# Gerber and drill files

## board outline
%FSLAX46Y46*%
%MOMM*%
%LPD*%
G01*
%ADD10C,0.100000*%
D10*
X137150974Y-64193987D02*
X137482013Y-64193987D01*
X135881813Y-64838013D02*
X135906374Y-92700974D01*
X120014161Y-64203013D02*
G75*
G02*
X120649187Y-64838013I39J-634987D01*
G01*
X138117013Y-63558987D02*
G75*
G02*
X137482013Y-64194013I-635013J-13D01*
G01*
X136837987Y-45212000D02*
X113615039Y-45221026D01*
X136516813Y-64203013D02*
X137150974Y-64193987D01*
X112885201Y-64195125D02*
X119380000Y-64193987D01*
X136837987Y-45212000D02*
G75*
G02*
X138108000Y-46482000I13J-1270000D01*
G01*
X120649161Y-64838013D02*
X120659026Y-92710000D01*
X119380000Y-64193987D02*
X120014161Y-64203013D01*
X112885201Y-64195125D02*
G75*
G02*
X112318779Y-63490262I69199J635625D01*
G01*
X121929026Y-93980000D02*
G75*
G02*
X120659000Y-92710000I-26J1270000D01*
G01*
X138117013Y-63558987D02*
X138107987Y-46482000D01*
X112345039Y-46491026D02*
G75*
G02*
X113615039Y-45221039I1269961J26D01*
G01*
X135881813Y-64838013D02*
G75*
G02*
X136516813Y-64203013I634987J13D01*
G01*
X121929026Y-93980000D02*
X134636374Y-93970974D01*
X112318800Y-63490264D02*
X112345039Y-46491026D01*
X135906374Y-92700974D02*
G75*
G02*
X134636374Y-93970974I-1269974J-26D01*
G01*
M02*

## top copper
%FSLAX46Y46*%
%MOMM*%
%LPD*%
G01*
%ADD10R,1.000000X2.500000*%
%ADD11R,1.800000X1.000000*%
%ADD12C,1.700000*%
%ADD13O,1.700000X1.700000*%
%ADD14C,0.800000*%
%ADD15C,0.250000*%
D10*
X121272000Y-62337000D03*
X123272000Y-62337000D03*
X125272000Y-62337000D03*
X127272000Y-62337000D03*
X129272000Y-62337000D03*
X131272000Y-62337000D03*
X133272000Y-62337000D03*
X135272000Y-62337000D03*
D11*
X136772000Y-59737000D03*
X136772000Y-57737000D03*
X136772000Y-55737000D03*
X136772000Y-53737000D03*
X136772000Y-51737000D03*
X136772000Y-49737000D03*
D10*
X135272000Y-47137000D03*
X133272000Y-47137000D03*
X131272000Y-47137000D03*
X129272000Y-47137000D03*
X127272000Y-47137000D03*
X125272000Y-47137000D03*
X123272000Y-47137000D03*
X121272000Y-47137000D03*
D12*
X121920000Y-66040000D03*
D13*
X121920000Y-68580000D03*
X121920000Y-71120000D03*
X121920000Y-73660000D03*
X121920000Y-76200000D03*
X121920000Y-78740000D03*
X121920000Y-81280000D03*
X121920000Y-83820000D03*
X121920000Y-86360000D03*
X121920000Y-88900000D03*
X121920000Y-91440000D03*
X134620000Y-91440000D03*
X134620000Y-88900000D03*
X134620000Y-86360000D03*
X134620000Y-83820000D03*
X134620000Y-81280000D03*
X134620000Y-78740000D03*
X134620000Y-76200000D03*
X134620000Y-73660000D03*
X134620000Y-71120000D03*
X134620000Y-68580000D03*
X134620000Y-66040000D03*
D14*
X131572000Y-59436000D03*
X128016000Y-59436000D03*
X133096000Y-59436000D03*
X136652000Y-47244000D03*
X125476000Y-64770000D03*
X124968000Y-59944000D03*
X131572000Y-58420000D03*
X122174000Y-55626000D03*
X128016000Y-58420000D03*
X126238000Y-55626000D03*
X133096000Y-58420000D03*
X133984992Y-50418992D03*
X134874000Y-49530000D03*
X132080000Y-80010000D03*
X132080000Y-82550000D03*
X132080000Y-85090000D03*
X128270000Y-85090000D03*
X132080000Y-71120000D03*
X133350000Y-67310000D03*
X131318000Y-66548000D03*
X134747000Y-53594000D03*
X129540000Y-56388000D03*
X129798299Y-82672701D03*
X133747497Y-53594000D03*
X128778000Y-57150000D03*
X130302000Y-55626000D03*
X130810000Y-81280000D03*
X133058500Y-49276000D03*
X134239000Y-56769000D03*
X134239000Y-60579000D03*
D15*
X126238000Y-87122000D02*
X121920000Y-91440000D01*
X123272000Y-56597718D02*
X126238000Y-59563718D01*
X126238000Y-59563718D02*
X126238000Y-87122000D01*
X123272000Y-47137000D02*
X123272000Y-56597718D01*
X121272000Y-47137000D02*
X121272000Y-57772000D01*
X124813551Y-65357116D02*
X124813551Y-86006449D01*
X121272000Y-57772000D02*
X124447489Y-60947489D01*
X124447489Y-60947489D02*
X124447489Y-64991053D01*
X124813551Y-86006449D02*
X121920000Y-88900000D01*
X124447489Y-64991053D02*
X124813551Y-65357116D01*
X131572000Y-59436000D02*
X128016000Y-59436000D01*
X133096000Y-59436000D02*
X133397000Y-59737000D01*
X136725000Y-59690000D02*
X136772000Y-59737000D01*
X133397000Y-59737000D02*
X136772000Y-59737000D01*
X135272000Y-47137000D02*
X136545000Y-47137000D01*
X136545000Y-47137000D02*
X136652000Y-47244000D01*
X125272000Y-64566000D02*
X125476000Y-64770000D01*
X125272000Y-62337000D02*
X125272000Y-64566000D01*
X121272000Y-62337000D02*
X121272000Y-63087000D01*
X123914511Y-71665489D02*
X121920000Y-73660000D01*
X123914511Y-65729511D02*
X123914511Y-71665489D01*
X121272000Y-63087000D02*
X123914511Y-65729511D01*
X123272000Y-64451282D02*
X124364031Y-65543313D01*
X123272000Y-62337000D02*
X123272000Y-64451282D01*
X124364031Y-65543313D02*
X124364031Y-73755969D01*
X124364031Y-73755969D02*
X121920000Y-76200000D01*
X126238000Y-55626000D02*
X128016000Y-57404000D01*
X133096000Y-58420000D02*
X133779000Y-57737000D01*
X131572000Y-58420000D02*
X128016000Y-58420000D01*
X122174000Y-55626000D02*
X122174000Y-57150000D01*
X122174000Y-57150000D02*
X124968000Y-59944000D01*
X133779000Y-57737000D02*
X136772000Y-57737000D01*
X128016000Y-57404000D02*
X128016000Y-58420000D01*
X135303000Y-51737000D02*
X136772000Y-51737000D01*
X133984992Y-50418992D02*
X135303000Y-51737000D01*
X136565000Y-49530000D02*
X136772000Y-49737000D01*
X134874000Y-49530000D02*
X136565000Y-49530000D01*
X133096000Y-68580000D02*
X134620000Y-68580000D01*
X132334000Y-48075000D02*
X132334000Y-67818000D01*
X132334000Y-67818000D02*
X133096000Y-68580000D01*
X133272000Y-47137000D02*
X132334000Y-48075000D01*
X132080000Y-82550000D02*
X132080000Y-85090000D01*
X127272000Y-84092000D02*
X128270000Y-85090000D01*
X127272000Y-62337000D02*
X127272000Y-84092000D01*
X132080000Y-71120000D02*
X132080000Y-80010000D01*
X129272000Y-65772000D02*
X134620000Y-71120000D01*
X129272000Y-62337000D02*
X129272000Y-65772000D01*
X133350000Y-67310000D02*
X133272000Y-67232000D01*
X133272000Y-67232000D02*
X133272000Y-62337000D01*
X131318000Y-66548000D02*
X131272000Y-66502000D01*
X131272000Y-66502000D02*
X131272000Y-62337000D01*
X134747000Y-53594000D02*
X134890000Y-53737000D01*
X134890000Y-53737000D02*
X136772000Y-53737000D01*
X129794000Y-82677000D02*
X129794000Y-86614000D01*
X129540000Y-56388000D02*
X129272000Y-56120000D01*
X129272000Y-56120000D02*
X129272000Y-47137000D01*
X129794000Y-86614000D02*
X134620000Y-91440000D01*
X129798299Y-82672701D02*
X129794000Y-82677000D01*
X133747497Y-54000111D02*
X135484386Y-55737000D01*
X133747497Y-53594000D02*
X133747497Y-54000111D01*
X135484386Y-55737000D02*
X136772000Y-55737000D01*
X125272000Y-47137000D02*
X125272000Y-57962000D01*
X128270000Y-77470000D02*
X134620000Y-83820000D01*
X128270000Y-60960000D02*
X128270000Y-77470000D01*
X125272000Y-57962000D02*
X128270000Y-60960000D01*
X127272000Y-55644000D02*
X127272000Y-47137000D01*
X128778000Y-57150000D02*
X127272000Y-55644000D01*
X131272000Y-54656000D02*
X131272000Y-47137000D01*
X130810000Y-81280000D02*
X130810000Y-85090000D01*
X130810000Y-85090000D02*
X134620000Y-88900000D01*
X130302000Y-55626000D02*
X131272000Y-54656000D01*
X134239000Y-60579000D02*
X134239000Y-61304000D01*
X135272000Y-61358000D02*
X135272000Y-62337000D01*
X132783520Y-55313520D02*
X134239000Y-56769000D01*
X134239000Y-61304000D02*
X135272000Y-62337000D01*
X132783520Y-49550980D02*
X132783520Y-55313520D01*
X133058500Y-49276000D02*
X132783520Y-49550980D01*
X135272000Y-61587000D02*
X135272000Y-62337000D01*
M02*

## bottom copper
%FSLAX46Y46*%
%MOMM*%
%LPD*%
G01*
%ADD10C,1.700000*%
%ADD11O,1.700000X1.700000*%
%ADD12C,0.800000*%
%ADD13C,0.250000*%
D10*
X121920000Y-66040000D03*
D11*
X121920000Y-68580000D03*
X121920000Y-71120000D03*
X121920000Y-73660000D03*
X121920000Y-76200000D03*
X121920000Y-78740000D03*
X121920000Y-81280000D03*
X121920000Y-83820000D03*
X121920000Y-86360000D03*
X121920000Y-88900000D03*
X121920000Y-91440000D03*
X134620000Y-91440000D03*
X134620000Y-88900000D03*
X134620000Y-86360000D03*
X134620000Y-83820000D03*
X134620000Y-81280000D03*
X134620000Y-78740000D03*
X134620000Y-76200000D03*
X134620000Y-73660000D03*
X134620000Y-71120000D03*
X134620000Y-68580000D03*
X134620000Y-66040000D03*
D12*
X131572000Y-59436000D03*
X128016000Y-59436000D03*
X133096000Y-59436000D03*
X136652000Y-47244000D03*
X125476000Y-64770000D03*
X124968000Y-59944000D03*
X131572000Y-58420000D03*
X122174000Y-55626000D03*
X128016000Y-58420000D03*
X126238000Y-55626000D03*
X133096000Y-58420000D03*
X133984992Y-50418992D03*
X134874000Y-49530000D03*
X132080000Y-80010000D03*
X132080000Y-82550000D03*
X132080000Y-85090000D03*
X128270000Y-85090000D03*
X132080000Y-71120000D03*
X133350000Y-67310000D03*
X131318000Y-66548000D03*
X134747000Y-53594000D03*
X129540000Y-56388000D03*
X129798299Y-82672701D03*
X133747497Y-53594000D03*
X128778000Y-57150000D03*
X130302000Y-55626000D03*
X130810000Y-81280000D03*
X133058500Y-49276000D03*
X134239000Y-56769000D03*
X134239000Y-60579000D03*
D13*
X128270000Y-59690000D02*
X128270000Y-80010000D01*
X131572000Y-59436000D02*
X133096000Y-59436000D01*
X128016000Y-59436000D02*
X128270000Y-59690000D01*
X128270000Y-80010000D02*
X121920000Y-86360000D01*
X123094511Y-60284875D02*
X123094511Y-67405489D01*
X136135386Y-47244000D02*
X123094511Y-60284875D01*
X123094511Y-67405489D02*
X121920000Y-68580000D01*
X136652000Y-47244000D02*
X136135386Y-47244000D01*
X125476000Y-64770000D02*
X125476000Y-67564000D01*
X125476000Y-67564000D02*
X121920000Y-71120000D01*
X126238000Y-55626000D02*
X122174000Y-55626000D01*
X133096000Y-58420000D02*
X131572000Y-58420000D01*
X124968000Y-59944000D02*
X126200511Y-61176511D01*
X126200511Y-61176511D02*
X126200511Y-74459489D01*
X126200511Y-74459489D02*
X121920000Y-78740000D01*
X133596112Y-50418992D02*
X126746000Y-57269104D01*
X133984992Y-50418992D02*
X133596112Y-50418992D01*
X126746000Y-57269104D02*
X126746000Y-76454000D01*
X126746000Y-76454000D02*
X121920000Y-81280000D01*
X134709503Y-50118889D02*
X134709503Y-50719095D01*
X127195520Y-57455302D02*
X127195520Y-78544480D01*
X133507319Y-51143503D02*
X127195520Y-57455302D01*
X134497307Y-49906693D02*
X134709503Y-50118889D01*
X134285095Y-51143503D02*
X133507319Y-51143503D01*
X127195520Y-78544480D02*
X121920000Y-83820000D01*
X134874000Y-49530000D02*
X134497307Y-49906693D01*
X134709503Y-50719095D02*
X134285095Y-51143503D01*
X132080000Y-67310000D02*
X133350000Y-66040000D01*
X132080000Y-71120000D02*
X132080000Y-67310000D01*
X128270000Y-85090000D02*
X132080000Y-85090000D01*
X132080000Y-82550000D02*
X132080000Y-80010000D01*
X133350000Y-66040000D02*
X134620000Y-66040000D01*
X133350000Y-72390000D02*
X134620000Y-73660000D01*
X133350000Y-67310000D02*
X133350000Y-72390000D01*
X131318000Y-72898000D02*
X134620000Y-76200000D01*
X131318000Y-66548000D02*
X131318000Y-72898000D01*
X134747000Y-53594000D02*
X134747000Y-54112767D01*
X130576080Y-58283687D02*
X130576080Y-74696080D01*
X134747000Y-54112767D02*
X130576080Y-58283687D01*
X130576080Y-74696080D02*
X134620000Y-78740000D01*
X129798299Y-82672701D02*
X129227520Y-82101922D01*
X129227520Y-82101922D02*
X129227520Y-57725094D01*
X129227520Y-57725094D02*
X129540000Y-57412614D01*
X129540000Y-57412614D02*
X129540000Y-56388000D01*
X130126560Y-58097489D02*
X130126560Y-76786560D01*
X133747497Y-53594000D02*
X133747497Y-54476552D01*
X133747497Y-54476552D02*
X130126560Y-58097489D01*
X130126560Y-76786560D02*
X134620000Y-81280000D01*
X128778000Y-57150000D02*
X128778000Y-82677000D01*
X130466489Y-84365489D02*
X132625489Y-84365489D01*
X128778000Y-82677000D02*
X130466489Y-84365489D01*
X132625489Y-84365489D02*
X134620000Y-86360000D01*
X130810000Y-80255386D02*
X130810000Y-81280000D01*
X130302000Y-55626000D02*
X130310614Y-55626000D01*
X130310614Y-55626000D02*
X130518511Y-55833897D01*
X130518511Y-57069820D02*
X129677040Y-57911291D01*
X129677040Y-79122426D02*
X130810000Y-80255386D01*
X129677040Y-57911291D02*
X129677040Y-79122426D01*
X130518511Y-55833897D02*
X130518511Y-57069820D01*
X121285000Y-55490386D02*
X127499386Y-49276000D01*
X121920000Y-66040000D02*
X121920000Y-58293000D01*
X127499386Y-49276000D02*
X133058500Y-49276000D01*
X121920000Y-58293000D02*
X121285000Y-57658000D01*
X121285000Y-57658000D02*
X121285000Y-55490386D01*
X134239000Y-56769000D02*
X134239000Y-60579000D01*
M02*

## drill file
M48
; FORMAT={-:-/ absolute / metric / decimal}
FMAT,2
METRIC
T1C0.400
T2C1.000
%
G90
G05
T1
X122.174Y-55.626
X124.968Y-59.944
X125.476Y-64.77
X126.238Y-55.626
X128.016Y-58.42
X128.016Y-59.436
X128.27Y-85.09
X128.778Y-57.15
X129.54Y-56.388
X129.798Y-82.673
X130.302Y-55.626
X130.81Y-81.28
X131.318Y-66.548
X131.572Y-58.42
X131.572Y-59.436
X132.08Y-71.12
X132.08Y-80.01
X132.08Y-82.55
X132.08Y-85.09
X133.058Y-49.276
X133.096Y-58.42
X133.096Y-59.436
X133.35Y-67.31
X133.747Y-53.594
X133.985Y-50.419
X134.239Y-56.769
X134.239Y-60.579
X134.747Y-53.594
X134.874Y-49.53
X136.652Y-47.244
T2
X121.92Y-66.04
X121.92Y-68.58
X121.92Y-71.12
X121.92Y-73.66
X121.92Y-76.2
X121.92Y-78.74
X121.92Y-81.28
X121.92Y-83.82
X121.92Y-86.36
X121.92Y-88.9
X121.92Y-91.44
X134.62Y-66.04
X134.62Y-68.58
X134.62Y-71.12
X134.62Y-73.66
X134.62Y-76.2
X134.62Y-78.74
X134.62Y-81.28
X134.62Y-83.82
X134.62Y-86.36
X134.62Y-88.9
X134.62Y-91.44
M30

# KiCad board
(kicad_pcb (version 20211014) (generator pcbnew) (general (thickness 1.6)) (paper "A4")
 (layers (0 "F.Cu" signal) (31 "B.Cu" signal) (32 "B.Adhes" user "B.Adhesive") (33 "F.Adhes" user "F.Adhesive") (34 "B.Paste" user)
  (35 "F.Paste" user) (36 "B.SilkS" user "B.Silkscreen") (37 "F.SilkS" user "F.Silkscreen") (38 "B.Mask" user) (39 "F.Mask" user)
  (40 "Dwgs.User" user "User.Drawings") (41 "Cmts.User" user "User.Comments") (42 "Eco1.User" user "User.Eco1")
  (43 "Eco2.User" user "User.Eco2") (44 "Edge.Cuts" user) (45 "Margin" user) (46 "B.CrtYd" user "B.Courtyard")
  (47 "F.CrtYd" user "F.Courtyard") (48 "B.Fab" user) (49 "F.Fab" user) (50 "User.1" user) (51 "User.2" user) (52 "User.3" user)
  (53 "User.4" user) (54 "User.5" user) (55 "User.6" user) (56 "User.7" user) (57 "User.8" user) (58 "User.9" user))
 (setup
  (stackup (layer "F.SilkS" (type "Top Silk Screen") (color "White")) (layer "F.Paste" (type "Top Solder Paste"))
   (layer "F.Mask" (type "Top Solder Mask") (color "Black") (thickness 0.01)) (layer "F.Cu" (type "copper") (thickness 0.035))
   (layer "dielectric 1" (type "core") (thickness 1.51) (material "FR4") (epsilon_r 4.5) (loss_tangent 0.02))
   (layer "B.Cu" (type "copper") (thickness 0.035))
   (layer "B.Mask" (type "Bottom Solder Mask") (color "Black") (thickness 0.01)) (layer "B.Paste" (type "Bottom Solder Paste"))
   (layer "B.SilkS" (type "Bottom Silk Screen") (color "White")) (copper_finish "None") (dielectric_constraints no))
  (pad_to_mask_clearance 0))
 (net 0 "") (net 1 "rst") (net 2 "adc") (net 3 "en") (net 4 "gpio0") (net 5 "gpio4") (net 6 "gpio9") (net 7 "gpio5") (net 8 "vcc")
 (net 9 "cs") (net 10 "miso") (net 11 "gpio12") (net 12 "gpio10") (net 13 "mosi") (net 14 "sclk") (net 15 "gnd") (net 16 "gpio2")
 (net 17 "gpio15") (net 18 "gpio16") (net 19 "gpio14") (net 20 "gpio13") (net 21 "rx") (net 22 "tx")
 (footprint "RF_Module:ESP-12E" (layer "F.Cu") (at 124.772 54.737 90)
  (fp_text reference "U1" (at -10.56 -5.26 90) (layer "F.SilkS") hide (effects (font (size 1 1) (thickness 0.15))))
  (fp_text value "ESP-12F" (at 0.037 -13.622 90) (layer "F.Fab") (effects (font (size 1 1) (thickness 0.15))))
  (pad "1" smd rect (at -7.6 -3.5 90) (size 2.5 1) (layers "F.Cu" "F.Paste" "F.Mask") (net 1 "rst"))
  (pad "2" smd rect (at -7.6 -1.5 90) (size 2.5 1) (layers "F.Cu" "F.Paste" "F.Mask") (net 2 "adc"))
  (pad "3" smd rect (at -7.6 0.5 90) (size 2.5 1) (layers "F.Cu" "F.Paste" "F.Mask") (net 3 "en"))
  (pad "4" smd rect (at -7.6 2.5 90) (size 2.5 1) (layers "F.Cu" "F.Paste" "F.Mask") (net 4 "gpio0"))
  (pad "5" smd rect (at -7.6 4.5 90) (size 2.5 1) (layers "F.Cu" "F.Paste" "F.Mask") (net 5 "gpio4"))
  (pad "6" smd rect (at -7.6 6.5 90) (size 2.5 1) (layers "F.Cu" "F.Paste" "F.Mask") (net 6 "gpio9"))
  (pad "7" smd rect (at -7.6 8.5 90) (size 2.5 1) (layers "F.Cu" "F.Paste" "F.Mask") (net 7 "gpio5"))
  (pad "8" smd rect (at -7.6 10.5 90) (size 2.5 1) (layers "F.Cu" "F.Paste" "F.Mask") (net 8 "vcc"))
  (pad "9" smd rect (at -5 12 90) (size 1 1.8) (layers "F.Cu" "F.Paste" "F.Mask") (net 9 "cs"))
  (pad "10" smd rect (at -3 12 90) (size 1 1.8) (layers "F.Cu" "F.Paste" "F.Mask") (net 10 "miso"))
  (pad "11" smd rect (at -1 12 90) (size 1 1.8) (layers "F.Cu" "F.Paste" "F.Mask") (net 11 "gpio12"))
  (pad "12" smd rect (at 1 12 90) (size 1 1.8) (layers "F.Cu" "F.Paste" "F.Mask") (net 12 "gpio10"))
  (pad "13" smd rect (at 3 12 90) (size 1 1.8) (layers "F.Cu" "F.Paste" "F.Mask") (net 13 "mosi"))
  (pad "14" smd rect (at 5 12 90) (size 1 1.8) (layers "F.Cu" "F.Paste" "F.Mask") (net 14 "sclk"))
  (pad "15" smd rect (at 7.6 10.5 90) (size 2.5 1) (layers "F.Cu" "F.Paste" "F.Mask") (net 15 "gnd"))
  (pad "16" smd rect (at 7.6 8.5 90) (size 2.5 1) (layers "F.Cu" "F.Paste" "F.Mask") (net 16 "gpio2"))
  (pad "17" smd rect (at 7.6 6.5 90) (size 2.5 1) (layers "F.Cu" "F.Paste" "F.Mask") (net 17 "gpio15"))
  (pad "18" smd rect (at 7.6 4.5 90) (size 2.5 1) (layers "F.Cu" "F.Paste" "F.Mask") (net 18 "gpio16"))
  (pad "19" smd rect (at 7.6 2.5 90) (size 2.5 1) (layers "F.Cu" "F.Paste" "F.Mask") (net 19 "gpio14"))
  (pad "20" smd rect (at 7.6 0.5 90) (size 2.5 1) (layers "F.Cu" "F.Paste" "F.Mask") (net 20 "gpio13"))
  (pad "21" smd rect (at 7.6 -1.5 90) (size 2.5 1) (layers "F.Cu" "F.Paste" "F.Mask") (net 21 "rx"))
  (pad "22" smd rect (at 7.6 -3.5 90) (size 2.5 1) (layers "F.Cu" "F.Paste" "F.Mask") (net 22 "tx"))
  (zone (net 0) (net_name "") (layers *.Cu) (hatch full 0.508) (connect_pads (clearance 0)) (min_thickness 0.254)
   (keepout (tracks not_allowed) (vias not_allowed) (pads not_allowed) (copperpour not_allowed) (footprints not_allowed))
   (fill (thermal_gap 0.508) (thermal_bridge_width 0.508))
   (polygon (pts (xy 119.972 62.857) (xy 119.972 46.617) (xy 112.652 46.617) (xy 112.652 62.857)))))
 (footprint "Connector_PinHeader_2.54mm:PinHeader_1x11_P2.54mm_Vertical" (layer "B.Cu") (at 121.92 66.04 180)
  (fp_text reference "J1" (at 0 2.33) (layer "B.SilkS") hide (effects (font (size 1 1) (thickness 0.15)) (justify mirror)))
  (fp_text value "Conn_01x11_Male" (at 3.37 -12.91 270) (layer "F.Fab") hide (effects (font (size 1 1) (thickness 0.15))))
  (pad "1" thru_hole circle (at 0 0 180) (size 1.7 1.7) (drill 1) (layers *.Cu *.Mask) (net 8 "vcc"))
  (pad "2" thru_hole oval (at 0 -2.54 180) (size 1.7 1.7) (drill 1) (layers *.Cu *.Mask) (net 15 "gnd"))
  (pad "3" thru_hole oval (at 0 -5.08 180) (size 1.7 1.7) (drill 1) (layers *.Cu *.Mask) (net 3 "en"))
  (pad "4" thru_hole oval (at 0 -7.62 180) (size 1.7 1.7) (drill 1) (layers *.Cu *.Mask) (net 1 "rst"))
  (pad "5" thru_hole oval (at 0 -10.16 180) (size 1.7 1.7) (drill 1) (layers *.Cu *.Mask) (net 2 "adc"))
  (pad "6" thru_hole oval (at 0 -12.7 180) (size 1.7 1.7) (drill 1) (layers *.Cu *.Mask) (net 10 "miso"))
  (pad "7" thru_hole oval (at 0 -15.24 180) (size 1.7 1.7) (drill 1) (layers *.Cu *.Mask) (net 13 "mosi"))
  (pad "8" thru_hole oval (at 0 -17.78 180) (size 1.7 1.7) (drill 1) (layers *.Cu *.Mask) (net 14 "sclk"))
  (pad "9" thru_hole oval (at 0 -20.32 180) (size 1.7 1.7) (drill 1) (layers *.Cu *.Mask) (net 9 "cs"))
  (pad "10" thru_hole oval (at 0 -22.86 180) (size 1.7 1.7) (drill 1) (layers *.Cu *.Mask) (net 22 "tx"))
  (pad "11" thru_hole oval (at 0 -25.4 180) (size 1.7 1.7) (drill 1) (layers *.Cu *.Mask) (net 21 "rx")))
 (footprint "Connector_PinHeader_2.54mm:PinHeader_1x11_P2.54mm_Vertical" (layer "B.Cu") (at 134.62 91.44)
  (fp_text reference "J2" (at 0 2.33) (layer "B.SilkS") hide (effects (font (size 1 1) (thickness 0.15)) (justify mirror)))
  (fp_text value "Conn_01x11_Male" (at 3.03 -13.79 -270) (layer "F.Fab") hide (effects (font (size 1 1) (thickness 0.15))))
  (pad "1" thru_hole oval (at 0 0) (size 1.7 1.7) (drill 1) (layers *.Cu *.Mask) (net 18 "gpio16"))
  (pad "2" thru_hole oval (at 0 -2.54) (size 1.7 1.7) (drill 1) (layers *.Cu *.Mask) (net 17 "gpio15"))
  (pad "3" thru_hole oval (at 0 -5.08) (size 1.7 1.7) (drill 1) (layers *.Cu *.Mask) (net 19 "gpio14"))
  (pad "4" thru_hole oval (at 0 -7.62) (size 1.7 1.7) (drill 1) (layers *.Cu *.Mask) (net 20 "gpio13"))
  (pad "5" thru_hole oval (at 0 -10.16) (size 1.7 1.7) (drill 1) (layers *.Cu *.Mask) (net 11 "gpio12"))
  (pad "6" thru_hole oval (at 0 -12.7) (size 1.7 1.7) (drill 1) (layers *.Cu *.Mask) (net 12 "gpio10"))
  (pad "7" thru_hole oval (at 0 -15.24) (size 1.7 1.7) (drill 1) (layers *.Cu *.Mask) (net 6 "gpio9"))
  (pad "8" thru_hole oval (at 0 -17.78) (size 1.7 1.7) (drill 1) (layers *.Cu *.Mask) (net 7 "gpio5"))
  (pad "9" thru_hole oval (at 0 -20.32) (size 1.7 1.7) (drill 1) (layers *.Cu *.Mask) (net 5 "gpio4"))
  (pad "10" thru_hole oval (at 0 -22.86) (size 1.7 1.7) (drill 1) (layers *.Cu *.Mask) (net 16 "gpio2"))
  (pad "11" thru_hole oval (at 0 -25.4) (size 1.7 1.7) (drill 1) (layers *.Cu *.Mask) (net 4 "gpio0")))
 (gr_line (start 137.150974 64.193987) (end 137.482013 64.193987) (layer "Edge.Cuts") (width 0.1))
 (gr_line (start 135.881813 64.838013) (end 135.906374 92.700974) (layer "Edge.Cuts") (width 0.1))
 (gr_arc (start 120.014161 64.203013) (mid 120.463174 64.389) (end 120.649161 64.838013) (layer "Edge.Cuts") (width 0.1))
 (gr_arc (start 138.117013 63.558987) (mid 137.931026 64.008) (end 137.482013 64.193987) (layer "Edge.Cuts") (width 0.1))
 (gr_line (start 136.837987 45.212) (end 113.615039 45.221026) (layer "Edge.Cuts") (width 0.1))
 (gr_line (start 136.516813 64.203013) (end 137.150974 64.193987) (layer "Edge.Cuts") (width 0.1))
 (gr_line (start 112.885201 64.195125) (end 119.38 64.193987) (layer "Edge.Cuts") (width 0.1))
 (gr_arc (start 136.837987 45.212) (mid 137.736013 45.583974) (end 138.107987 46.482) (layer "Edge.Cuts") (width 0.1))
 (gr_line (start 120.649161 64.838013) (end 120.659026 92.71) (layer "Edge.Cuts") (width 0.1))
 (gr_line (start 119.38 64.193987) (end 120.014161 64.203013) (layer "Edge.Cuts") (width 0.1))
 (gr_arc (start 112.885201 64.195125) (mid 112.456019 63.96) (end 112.3188 63.490264) (layer "Edge.Cuts") (width 0.1))
 (gr_arc (start 121.929026 93.98) (mid 121.031 93.608026) (end 120.659026 92.71) (layer "Edge.Cuts") (width 0.1))
 (gr_line (start 138.117013 63.558987) (end 138.107987 46.482) (layer "Edge.Cuts") (width 0.1))
 (gr_arc (start 112.345039 46.491026) (mid 112.717013 45.593) (end 113.615039 45.221026) (layer "Edge.Cuts") (width 0.1))
 (gr_arc (start 135.881813 64.838013) (mid 136.0678 64.389) (end 136.516813 64.203013) (layer "Edge.Cuts") (width 0.1))
 (gr_line (start 121.929026 93.98) (end 134.636374 93.970974) (layer "Edge.Cuts") (width 0.1))
 (gr_line (start 112.3188 63.490264) (end 112.345039 46.491026) (layer "Edge.Cuts") (width 0.1))
 (gr_arc (start 135.906374 92.700974) (mid 135.5344 93.599) (end 134.636374 93.970974) (layer "Edge.Cuts") (width 0.1))
 (segment (start 126.238 87.122) (end 121.92 91.44) (width 0.25) (layer "F.Cu") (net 21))
 (segment (start 123.272 56.597718) (end 126.238 59.563718) (width 0.25) (layer "F.Cu") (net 21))
 (segment (start 126.238 59.563718) (end 126.238 87.122) (width 0.25) (layer "F.Cu") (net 21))
 (segment (start 123.272 47.137) (end 123.272 56.597718) (width 0.25) (layer "F.Cu") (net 21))
 (segment (start 121.272 47.137) (end 121.272 57.772) (width 0.25) (layer "F.Cu") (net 22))
 (segment (start 124.813551 65.357116) (end 124.813551 86.006449) (width 0.25) (layer "F.Cu") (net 22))
 (segment (start 121.272 57.772) (end 124.447489 60.947489) (width 0.25) (layer "F.Cu") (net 22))
 (segment (start 124.447489 60.947489) (end 124.447489 64.991053) (width 0.25) (layer "F.Cu") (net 22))
 (segment (start 124.813551 86.006449) (end 121.92 88.9) (width 0.25) (layer "F.Cu") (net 22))
 (segment (start 124.447489 64.991053) (end 124.813551 65.357116) (width 0.25) (layer "F.Cu") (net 22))
 (segment (start 131.572 59.436) (end 128.016 59.436) (width 0.25) (layer "F.Cu") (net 9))
 (segment (start 133.096 59.436) (end 133.397 59.737) (width 0.25) (layer "F.Cu") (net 9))
 (segment (start 136.725 59.69) (end 136.772 59.737) (width 0.25) (layer "F.Cu") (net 9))
 (segment (start 133.397 59.737) (end 136.772 59.737) (width 0.25) (layer "F.Cu") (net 9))
 (via (at 131.572 59.436) (size 0.8) (drill 0.4) (layers "F.Cu" "B.Cu") (free) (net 9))
 (via (at 128.016 59.436) (size 0.8) (drill 0.4) (layers "F.Cu" "B.Cu") (free) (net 9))
 (via (at 133.096 59.436) (size 0.8) (drill 0.4) (layers "F.Cu" "B.Cu") (free) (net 9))
 (segment (start 128.27 59.69) (end 128.27 80.01) (width 0.25) (layer "B.Cu") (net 9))
 (segment (start 131.572 59.436) (end 133.096 59.436) (width 0.25) (layer "B.Cu") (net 9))
 (segment (start 128.016 59.436) (end 128.27 59.69) (width 0.25) (layer "B.Cu") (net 9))
 (segment (start 128.27 80.01) (end 121.92 86.36) (width 0.25) (layer "B.Cu") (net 9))
 (segment (start 135.272 47.137) (end 136.545 47.137) (width 0.25) (layer "F.Cu") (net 15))
 (segment (start 136.545 47.137) (end 136.652 47.244) (width 0.25) (layer "F.Cu") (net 15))
 (via (at 136.652 47.244) (size 0.8) (drill 0.4) (layers "F.Cu" "B.Cu") (free) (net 15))
 (segment (start 123.094511 60.284875) (end 123.094511 67.405489) (width 0.25) (layer "B.Cu") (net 15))
 (segment (start 136.135386 47.244) (end 123.094511 60.284875) (width 0.25) (layer "B.Cu") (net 15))
 (segment (start 123.094511 67.405489) (end 121.92 68.58) (width 0.25) (layer "B.Cu") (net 15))
 (segment (start 136.652 47.244) (end 136.135386 47.244) (width 0.25) (layer "B.Cu") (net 15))
 (segment (start 125.272 64.566) (end 125.476 64.77) (width 0.25) (layer "F.Cu") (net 3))
 (segment (start 125.272 62.337) (end 125.272 64.566) (width 0.25) (layer "F.Cu") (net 3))
 (via (at 125.476 64.77) (size 0.8) (drill 0.4) (layers "F.Cu" "B.Cu") (free) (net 3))
 (segment (start 125.476 64.77) (end 125.476 67.564) (width 0.25) (layer "B.Cu") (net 3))
 (segment (start 125.476 67.564) (end 121.92 71.12) (width 0.25) (layer "B.Cu") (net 3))
 (segment (start 121.272 62.337) (end 121.272 63.087) (width 0.25) (layer "F.Cu") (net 1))
 (segment (start 123.914511 71.665489) (end 121.92 73.66) (width 0.25) (layer "F.Cu") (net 1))
 (segment (start 123.914511 65.729511) (end 123.914511 71.665489) (width 0.25) (layer "F.Cu") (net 1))
 (segment (start 121.272 63.087) (end 123.914511 65.729511) (width 0.25) (layer "F.Cu") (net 1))
 (segment (start 123.272 64.451282) (end 124.364031 65.543313) (width 0.25) (layer "F.Cu") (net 2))
 (segment (start 123.272 62.337) (end 123.272 64.451282) (width 0.25) (layer "F.Cu") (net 2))
 (segment (start 124.364031 65.543313) (end 124.364031 73.755969) (width 0.25) (layer "F.Cu") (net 2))
 (segment (start 124.364031 73.755969) (end 121.92 76.2) (width 0.25) (layer "F.Cu") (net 2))
 (segment (start 126.238 55.626) (end 128.016 57.404) (width 0.25) (layer "F.Cu") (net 10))
 (segment (start 133.096 58.42) (end 133.779 57.737) (width 0.25) (layer "F.Cu") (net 10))
 (segment (start 131.572 58.42) (end 128.016 58.42) (width 0.25) (layer "F.Cu") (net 10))
 (segment (start 122.174 55.626) (end 122.174 57.15) (width 0.25) (layer "F.Cu") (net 10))
 (segment (start 122.174 57.15) (end 124.968 59.944) (width 0.25) (layer "F.Cu") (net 10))
 (segment (start 133.779 57.737) (end 136.772 57.737) (width 0.25) (layer "F.Cu") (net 10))
 (segment (start 128.016 57.404) (end 128.016 58.42) (width 0.25) (layer "F.Cu") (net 10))
 (via (at 124.968 59.944) (size 0.8) (drill 0.4) (layers "F.Cu" "B.Cu") (free) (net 10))
 (via (at 131.572 58.42) (size 0.8) (drill 0.4) (layers "F.Cu" "B.Cu") (free) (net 10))
 (via (at 122.174 55.626) (size 0.8) (drill 0.4) (layers "F.Cu" "B.Cu") (free) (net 10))
 (via (at 128.016 58.42) (size 0.8) (drill 0.4) (layers "F.Cu" "B.Cu") (free) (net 10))
 (via (at 126.238 55.626) (size 0.8) (drill 0.4) (layers "F.Cu" "B.Cu") (free) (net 10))
 (via (at 133.096 58.42) (size 0.8) (drill 0.4) (layers "F.Cu" "B.Cu") (free) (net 10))
 (segment (start 126.238 55.626) (end 122.174 55.626) (width 0.25) (layer "B.Cu") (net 10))
 (segment (start 133.096 58.42) (end 131.572 58.42) (width 0.25) (layer "B.Cu") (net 10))
 (segment (start 124.968 59.944) (end 126.200511 61.176511) (width 0.25) (layer "B.Cu") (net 10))
 (segment (start 126.200511 61.176511) (end 126.200511 74.459489) (width 0.25) (layer "B.Cu") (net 10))
 (segment (start 126.200511 74.459489) (end 121.92 78.74) (width 0.25) (layer "B.Cu") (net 10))
 (segment (start 135.303 51.737) (end 136.772 51.737) (width 0.25) (layer "F.Cu") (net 13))
 (segment (start 133.984992 50.418992) (end 135.303 51.737) (width 0.25) (layer "F.Cu") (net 13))
 (via (at 133.984992 50.418992) (size 0.8) (drill 0.4) (layers "F.Cu" "B.Cu") (free) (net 13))
 (segment (start 133.596112 50.418992) (end 126.746 57.269104) (width 0.25) (layer "B.Cu") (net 13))
 (segment (start 133.984992 50.418992) (end 133.596112 50.418992) (width 0.25) (layer "B.Cu") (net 13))
 (segment (start 126.746 57.269104) (end 126.746 76.454) (width 0.25) (layer "B.Cu") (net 13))
 (segment (start 126.746 76.454) (end 121.92 81.28) (width 0.25) (layer "B.Cu") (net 13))
 (segment (start 136.565 49.53) (end 136.772 49.737) (width 0.25) (layer "F.Cu") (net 14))
 (segment (start 134.874 49.53) (end 136.565 49.53) (width 0.25) (layer "F.Cu") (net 14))
 (via (at 134.874 49.53) (size 0.8) (drill 0.4) (layers "F.Cu" "B.Cu") (free) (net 14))
 (segment (start 134.709503 50.118889) (end 134.709503 50.719095) (width 0.25) (layer "B.Cu") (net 14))
 (segment (start 127.19552 57.455302) (end 127.19552 78.54448) (width 0.25) (layer "B.Cu") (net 14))
 (segment (start 133.507319 51.143503) (end 127.19552 57.455302) (width 0.25) (layer "B.Cu") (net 14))
 (segment (start 134.497307 49.906693) (end 134.709503 50.118889) (width 0.25) (layer "B.Cu") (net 14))
 (segment (start 134.285095 51.143503) (end 133.507319 51.143503) (width 0.25) (layer "B.Cu") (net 14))
 (segment (start 127.19552 78.54448) (end 121.92 83.82) (width 0.25) (layer "B.Cu") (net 14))
 (segment (start 134.874 49.53) (end 134.497307 49.906693) (width 0.25) (layer "B.Cu") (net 14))
 (segment (start 134.709503 50.719095) (end 134.285095 51.143503) (width 0.25) (layer "B.Cu") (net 14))
 (segment (start 133.096 68.58) (end 134.62 68.58) (width 0.25) (layer "F.Cu") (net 16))
 (segment (start 132.334 48.075) (end 132.334 67.818) (width 0.25) (layer "F.Cu") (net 16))
 (segment (start 132.334 67.818) (end 133.096 68.58) (width 0.25) (layer "F.Cu") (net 16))
 (segment (start 133.272 47.137) (end 132.334 48.075) (width 0.25) (layer "F.Cu") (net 16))
 (segment (start 132.08 82.55) (end 132.08 85.09) (width 0.25) (layer "F.Cu") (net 4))
 (segment (start 127.272 84.092) (end 128.27 85.09) (width 0.25) (layer "F.Cu") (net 4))
 (segment (start 127.272 62.337) (end 127.272 84.092) (width 0.25) (layer "F.Cu") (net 4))
 (segment (start 132.08 71.12) (end 132.08 80.01) (width 0.25) (layer "F.Cu") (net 4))
 (via (at 132.08 80.01) (size 0.8) (drill 0.4) (layers "F.Cu" "B.Cu") (free) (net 4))
 (via (at 132.08 82.55) (size 0.8) (drill 0.4) (layers "F.Cu" "B.Cu") (free) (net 4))
 (via (at 132.08 85.09) (size 0.8) (drill 0.4) (layers "F.Cu" "B.Cu") (free) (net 4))
 (via (at 128.27 85.09) (size 0.8) (drill 0.4) (layers "F.Cu" "B.Cu") (free) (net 4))
 (via (at 132.08 71.12) (size 0.8) (drill 0.4) (layers "F.Cu" "B.Cu") (free) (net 4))
 (segment (start 132.08 67.31) (end 133.35 66.04) (width 0.25) (layer "B.Cu") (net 4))
 (segment (start 132.08 71.12) (end 132.08 67.31) (width 0.25) (layer "B.Cu") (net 4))
 (segment (start 128.27 85.09) (end 132.08 85.09) (width 0.25) (layer "B.Cu") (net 4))
 (segment (start 132.08 82.55) (end 132.08 80.01) (width 0.25) (layer "B.Cu") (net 4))
 (segment (start 133.35 66.04) (end 134.62 66.04) (width 0.25) (layer "B.Cu") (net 4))
 (segment (start 129.272 65.772) (end 134.62 71.12) (width 0.25) (layer "F.Cu") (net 5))
 (segment (start 129.272 62.337) (end 129.272 65.772) (width 0.25) (layer "F.Cu") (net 5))
 (segment (start 133.35 67.31) (end 133.272 67.232) (width 0.25) (layer "F.Cu") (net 7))
 (segment (start 133.272 67.232) (end 133.272 62.337) (width 0.25) (layer "F.Cu") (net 7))
 (via (at 133.35 67.31) (size 0.8) (drill 0.4) (layers "F.Cu" "B.Cu") (free) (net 7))
 (segment (start 133.35 72.39) (end 134.62 73.66) (width 0.25) (layer "B.Cu") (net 7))
 (segment (start 133.35 67.31) (end 133.35 72.39) (width 0.25) (layer "B.Cu") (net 7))
 (segment (start 131.318 66.548) (end 131.272 66.502) (width 0.25) (layer "F.Cu") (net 6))
 (segment (start 131.272 66.502) (end 131.272 62.337) (width 0.25) (layer "F.Cu") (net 6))
 (via (at 131.318 66.548) (size 0.8) (drill 0.4) (layers "F.Cu" "B.Cu") (free) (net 6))
 (segment (start 131.318 72.898) (end 134.62 76.2) (width 0.25) (layer "B.Cu") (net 6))
 (segment (start 131.318 66.548) (end 131.318 72.898) (width 0.25) (layer "B.Cu") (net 6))
 (segment (start 134.747 53.594) (end 134.89 53.737) (width 0.25) (layer "F.Cu") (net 12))
 (segment (start 134.89 53.737) (end 136.772 53.737) (width 0.25) (layer "F.Cu") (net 12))
 (via (at 134.747 53.594) (size 0.8) (drill 0.4) (layers "F.Cu" "B.Cu") (free) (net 12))
 (segment (start 134.747 53.594) (end 134.747 54.112767) (width 0.25) (layer "B.Cu") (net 12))
 (segment (start 130.57608 58.283687) (end 130.57608 74.69608) (width 0.25) (layer "B.Cu") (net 12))
 (segment (start 134.747 54.112767) (end 130.57608 58.283687) (width 0.25) (layer "B.Cu") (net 12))
 (segment (start 130.57608 74.69608) (end 134.62 78.74) (width 0.25) (layer "B.Cu") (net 12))
 (segment (start 129.794 82.677) (end 129.794 86.614) (width 0.25) (layer "F.Cu") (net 18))
 (segment (start 129.54 56.388) (end 129.272 56.12) (width 0.25) (layer "F.Cu") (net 18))
 (segment (start 129.272 56.12) (end 129.272 47.137) (width 0.25) (layer "F.Cu") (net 18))
 (segment (start 129.794 86.614) (end 134.62 91.44) (width 0.25) (layer "F.Cu") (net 18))
 (segment (start 129.798299 82.672701) (end 129.794 82.677) (width 0.25) (layer "F.Cu") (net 18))
 (via (at 129.54 56.388) (size 0.8) (drill 0.4) (layers "F.Cu" "B.Cu") (free) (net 18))
 (via (at 129.798299 82.672701) (size 0.8) (drill 0.4) (layers "F.Cu" "B.Cu") (free) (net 18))
 (segment (start 129.798299 82.672701) (end 129.22752 82.101922) (width 0.25) (layer "B.Cu") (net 18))
 (segment (start 129.22752 82.101922) (end 129.22752 57.725094) (width 0.25) (layer "B.Cu") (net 18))
 (segment (start 129.22752 57.725094) (end 129.54 57.412614) (width 0.25) (layer "B.Cu") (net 18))
 (segment (start 129.54 57.412614) (end 129.54 56.388) (width 0.25) (layer "B.Cu") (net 18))
 (segment (start 133.747497 54.000111) (end 135.484386 55.737) (width 0.25) (layer "F.Cu") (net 11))
 (segment (start 133.747497 53.594) (end 133.747497 54.000111) (width 0.25) (layer "F.Cu") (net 11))
 (segment (start 135.484386 55.737) (end 136.772 55.737) (width 0.25) (layer "F.Cu") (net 11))
 (via (at 133.747497 53.594) (size 0.8) (drill 0.4) (layers "F.Cu" "B.Cu") (free) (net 11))
 (segment (start 130.12656 58.097489) (end 130.12656 76.78656) (width 0.25) (layer "B.Cu") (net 11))
 (segment (start 133.747497 53.594) (end 133.747497 54.476552) (width 0.25) (layer "B.Cu") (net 11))
 (segment (start 133.747497 54.476552) (end 130.12656 58.097489) (width 0.25) (layer "B.Cu") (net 11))
 (segment (start 130.12656 76.78656) (end 134.62 81.28) (width 0.25) (layer "B.Cu") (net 11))
 (segment (start 125.272 47.137) (end 125.272 57.962) (width 0.25) (layer "F.Cu") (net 20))
 (segment (start 128.27 77.47) (end 134.62 83.82) (width 0.25) (layer "F.Cu") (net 20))
 (segment (start 128.27 60.96) (end 128.27 77.47) (width 0.25) (layer "F.Cu") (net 20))
 (segment (start 125.272 57.962) (end 128.27 60.96) (width 0.25) (layer "F.Cu") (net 20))
 (segment (start 127.272 55.644) (end 127.272 47.137) (width 0.25) (layer "F.Cu") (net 19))
 (segment (start 128.778 57.15) (end 127.272 55.644) (width 0.25) (layer "F.Cu") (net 19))
 (via (at 128.778 57.15) (size 0.8) (drill 0.4) (layers "F.Cu" "B.Cu") (free) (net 19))
 (segment (start 128.778 57.15) (end 128.778 82.677) (width 0.25) (layer "B.Cu") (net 19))
 (segment (start 130.466489 84.365489) (end 132.625489 84.365489) (width 0.25) (layer "B.Cu") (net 19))
 (segment (start 128.778 82.677) (end 130.466489 84.365489) (width 0.25) (layer "B.Cu") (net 19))
 (segment (start 132.625489 84.365489) (end 134.62 86.36) (width 0.25) (layer "B.Cu") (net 19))
 (segment (start 131.272 54.656) (end 131.272 47.137) (width 0.25) (layer "F.Cu") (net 17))
 (segment (start 130.81 81.28) (end 130.81 85.09) (width 0.25) (layer "F.Cu") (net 17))
 (segment (start 130.81 85.09) (end 134.62 88.9) (width 0.25) (layer "F.Cu") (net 17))
 (segment (start 130.302 55.626) (end 131.272 54.656) (width 0.25) (layer "F.Cu") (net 17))
 (via (at 130.302 55.626) (size 0.8) (drill 0.4) (layers "F.Cu" "B.Cu") (free) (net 17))
 (via (at 130.81 81.28) (size 0.8) (drill 0.4) (layers "F.Cu" "B.Cu") (free) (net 17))
 (segment (start 130.81 80.255386) (end 130.81 81.28) (width 0.25) (layer "B.Cu") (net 17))
 (segment (start 130.302 55.626) (end 130.310614 55.626) (width 0.25) (layer "B.Cu") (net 17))
 (segment (start 130.310614 55.626) (end 130.518511 55.833897) (width 0.25) (layer "B.Cu") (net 17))
 (segment (start 130.518511 57.06982) (end 129.67704 57.911291) (width 0.25) (layer "B.Cu") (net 17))
 (segment (start 129.67704 79.122426) (end 130.81 80.255386) (width 0.25) (layer "B.Cu") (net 17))
 (segment (start 129.67704 57.911291) (end 129.67704 79.122426) (width 0.25) (layer "B.Cu") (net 17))
 (segment (start 130.518511 55.833897) (end 130.518511 57.06982) (width 0.25) (layer "B.Cu") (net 17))
 (segment (start 134.239 60.579) (end 134.239 61.304) (width 0.25) (layer "F.Cu") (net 8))
 (segment (start 135.272 61.358) (end 135.272 62.337) (width 0.25) (layer "F.Cu") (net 8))
 (segment (start 132.78352 55.31352) (end 134.239 56.769) (width 0.25) (layer "F.Cu") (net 8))
 (segment (start 134.239 61.304) (end 135.272 62.337) (width 0.25) (layer "F.Cu") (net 8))
 (segment (start 132.78352 49.55098) (end 132.78352 55.31352) (width 0.25) (layer "F.Cu") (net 8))
 (segment (start 133.0585 49.276) (end 132.78352 49.55098) (width 0.25) (layer "F.Cu") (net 8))
 (segment (start 135.272 61.587) (end 135.272 62.337) (width 0.25) (layer "F.Cu") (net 8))
 (via (at 133.0585 49.276) (size 0.8) (drill 0.4) (layers "F.Cu" "B.Cu") (free) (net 8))
 (via (at 134.239 56.769) (size 0.8) (drill 0.4) (layers "F.Cu" "B.Cu") (free) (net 8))
 (via (at 134.239 60.579) (size 0.8) (drill 0.4) (layers "F.Cu" "B.Cu") (free) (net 8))
 (segment (start 121.285 55.490386) (end 127.499386 49.276) (width 0.25) (layer "B.Cu") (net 8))
 (segment (start 121.92 66.04) (end 121.92 58.293) (width 0.25) (layer "B.Cu") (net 8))
 (segment (start 127.499386 49.276) (end 133.0585 49.276) (width 0.25) (layer "B.Cu") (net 8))
 (segment (start 121.92 58.293) (end 121.285 57.658) (width 0.25) (layer "B.Cu") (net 8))
 (segment (start 121.285 57.658) (end 121.285 55.490386) (width 0.25) (layer "B.Cu") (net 8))
 (segment (start 134.239 56.769) (end 134.239 60.579) (width 0.25) (layer "B.Cu") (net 8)))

